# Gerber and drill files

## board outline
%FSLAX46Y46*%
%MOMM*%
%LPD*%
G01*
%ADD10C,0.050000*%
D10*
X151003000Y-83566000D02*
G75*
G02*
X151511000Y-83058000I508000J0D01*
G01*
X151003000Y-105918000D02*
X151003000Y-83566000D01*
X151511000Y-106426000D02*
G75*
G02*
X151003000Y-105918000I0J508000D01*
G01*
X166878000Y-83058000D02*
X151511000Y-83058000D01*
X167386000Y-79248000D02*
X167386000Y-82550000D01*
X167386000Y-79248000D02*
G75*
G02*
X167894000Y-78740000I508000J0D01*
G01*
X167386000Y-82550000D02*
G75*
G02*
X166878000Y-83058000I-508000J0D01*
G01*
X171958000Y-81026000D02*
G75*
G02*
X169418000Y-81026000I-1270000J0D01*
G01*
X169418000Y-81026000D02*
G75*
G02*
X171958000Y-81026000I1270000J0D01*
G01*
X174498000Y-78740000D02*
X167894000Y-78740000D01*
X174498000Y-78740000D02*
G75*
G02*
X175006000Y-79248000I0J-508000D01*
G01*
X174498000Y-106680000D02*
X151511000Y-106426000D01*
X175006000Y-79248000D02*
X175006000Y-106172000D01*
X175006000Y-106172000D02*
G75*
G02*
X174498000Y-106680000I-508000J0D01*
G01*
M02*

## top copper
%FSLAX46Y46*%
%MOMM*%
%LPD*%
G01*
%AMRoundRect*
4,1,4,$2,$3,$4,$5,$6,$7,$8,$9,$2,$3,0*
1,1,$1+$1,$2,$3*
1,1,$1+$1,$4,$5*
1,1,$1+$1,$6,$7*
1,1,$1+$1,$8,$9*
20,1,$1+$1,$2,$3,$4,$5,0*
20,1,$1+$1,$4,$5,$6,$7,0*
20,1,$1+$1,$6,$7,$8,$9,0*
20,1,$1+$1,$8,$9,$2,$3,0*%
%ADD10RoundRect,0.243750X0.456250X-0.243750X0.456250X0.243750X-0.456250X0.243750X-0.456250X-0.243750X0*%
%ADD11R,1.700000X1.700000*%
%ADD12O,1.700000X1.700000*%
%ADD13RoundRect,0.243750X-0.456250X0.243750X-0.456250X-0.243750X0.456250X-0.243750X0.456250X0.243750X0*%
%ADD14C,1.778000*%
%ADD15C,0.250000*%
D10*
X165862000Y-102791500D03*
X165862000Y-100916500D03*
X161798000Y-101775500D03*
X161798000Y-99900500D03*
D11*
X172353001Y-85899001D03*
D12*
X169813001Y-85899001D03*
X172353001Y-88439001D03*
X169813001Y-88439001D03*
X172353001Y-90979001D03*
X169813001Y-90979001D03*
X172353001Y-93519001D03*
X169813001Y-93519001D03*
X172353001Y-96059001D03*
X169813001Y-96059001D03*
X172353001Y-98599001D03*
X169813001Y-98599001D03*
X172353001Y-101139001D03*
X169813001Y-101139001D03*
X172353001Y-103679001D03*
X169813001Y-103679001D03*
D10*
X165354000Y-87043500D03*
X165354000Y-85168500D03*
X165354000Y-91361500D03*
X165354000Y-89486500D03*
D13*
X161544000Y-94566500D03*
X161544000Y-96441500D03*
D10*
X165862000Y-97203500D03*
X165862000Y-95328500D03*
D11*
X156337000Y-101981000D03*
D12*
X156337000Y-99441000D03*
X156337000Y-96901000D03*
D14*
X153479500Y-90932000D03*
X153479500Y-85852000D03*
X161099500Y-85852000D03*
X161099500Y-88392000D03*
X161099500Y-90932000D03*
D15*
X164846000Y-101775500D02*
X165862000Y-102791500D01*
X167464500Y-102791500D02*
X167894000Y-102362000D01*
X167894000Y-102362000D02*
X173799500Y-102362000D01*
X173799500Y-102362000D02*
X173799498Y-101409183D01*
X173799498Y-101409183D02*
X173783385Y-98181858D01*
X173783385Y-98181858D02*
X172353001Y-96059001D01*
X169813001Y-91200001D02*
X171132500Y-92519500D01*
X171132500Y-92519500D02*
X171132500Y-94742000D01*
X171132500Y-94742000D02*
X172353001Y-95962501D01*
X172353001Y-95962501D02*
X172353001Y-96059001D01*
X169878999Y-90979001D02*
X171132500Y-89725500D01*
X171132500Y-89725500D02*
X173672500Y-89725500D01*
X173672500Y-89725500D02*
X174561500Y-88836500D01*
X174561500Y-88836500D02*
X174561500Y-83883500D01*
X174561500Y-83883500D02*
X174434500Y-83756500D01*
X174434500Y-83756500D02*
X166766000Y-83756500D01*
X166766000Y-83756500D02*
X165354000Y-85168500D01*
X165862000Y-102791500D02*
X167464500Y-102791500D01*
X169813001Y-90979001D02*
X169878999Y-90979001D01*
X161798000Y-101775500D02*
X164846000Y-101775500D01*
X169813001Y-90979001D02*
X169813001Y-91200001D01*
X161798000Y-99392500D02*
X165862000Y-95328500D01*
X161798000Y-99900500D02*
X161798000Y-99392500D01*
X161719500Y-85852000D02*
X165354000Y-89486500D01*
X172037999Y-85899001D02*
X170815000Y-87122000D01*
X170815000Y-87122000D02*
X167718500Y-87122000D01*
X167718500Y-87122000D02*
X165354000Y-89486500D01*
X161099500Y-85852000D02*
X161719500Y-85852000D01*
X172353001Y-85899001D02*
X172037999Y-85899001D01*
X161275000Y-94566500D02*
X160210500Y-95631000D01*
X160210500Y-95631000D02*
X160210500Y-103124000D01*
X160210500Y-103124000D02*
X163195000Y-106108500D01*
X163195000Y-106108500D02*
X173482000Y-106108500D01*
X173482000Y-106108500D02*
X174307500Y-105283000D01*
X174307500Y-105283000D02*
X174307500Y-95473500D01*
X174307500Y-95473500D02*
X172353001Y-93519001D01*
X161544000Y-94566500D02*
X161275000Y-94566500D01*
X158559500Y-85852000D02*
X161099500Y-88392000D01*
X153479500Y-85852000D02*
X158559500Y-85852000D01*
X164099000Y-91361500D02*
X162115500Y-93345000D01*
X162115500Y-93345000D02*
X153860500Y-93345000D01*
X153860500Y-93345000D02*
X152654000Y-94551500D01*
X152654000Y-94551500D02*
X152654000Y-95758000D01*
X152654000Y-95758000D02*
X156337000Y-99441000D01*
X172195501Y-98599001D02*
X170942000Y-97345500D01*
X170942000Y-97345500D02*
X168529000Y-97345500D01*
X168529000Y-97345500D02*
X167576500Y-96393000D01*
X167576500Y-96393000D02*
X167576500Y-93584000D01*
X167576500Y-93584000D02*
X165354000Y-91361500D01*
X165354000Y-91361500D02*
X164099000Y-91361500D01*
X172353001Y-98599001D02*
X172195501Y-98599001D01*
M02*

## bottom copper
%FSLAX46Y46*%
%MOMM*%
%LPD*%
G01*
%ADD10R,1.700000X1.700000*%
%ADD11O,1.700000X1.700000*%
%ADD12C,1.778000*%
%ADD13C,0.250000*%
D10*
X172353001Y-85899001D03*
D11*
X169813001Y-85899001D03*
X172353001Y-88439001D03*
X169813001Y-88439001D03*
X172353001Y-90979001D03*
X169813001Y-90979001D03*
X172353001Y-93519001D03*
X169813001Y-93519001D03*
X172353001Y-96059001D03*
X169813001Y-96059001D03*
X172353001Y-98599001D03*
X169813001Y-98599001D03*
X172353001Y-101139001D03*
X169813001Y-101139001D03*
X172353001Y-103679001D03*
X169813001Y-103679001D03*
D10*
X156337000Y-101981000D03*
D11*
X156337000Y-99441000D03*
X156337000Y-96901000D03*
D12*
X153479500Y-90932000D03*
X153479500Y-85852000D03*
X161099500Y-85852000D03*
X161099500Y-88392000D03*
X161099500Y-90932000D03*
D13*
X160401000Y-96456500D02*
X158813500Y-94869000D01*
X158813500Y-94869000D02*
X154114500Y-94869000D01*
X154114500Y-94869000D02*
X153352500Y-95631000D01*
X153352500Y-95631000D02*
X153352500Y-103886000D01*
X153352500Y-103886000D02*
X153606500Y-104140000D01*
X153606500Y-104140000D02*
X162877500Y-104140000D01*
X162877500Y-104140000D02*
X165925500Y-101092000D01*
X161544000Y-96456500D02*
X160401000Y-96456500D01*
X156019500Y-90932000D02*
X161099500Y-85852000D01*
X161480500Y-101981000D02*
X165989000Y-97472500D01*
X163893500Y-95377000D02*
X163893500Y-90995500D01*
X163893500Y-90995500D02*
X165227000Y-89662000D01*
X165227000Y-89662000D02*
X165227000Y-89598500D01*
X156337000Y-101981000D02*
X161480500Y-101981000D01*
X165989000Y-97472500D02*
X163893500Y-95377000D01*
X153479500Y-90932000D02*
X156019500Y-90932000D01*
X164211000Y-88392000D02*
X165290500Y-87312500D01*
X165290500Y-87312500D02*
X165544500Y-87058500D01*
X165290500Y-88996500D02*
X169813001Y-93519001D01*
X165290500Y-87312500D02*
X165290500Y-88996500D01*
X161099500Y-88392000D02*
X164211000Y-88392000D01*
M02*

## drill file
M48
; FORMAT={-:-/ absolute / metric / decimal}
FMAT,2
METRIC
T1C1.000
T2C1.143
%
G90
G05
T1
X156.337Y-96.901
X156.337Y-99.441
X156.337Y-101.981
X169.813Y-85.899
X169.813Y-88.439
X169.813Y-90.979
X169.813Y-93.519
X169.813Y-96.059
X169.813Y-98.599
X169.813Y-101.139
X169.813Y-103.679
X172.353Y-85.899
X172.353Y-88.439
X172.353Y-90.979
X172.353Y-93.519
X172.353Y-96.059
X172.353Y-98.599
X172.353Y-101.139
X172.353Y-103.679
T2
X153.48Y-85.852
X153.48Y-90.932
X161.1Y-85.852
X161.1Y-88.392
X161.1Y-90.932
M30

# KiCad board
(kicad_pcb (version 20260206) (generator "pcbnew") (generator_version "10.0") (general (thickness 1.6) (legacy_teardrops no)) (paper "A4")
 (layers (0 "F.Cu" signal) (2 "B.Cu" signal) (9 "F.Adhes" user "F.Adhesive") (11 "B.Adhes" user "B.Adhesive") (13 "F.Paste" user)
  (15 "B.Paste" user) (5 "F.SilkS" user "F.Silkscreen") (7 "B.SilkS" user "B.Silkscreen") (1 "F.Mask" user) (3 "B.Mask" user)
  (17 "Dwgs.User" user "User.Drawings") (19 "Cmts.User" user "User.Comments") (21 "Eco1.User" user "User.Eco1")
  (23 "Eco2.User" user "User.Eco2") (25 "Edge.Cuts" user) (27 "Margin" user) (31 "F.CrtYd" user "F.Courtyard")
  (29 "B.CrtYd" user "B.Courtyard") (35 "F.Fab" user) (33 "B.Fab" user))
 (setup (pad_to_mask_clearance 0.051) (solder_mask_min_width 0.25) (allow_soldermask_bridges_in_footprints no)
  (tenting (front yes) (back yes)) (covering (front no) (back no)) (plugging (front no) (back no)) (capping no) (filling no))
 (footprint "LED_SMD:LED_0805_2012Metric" (layer "F.Cu") (at 165.862 101.854 90)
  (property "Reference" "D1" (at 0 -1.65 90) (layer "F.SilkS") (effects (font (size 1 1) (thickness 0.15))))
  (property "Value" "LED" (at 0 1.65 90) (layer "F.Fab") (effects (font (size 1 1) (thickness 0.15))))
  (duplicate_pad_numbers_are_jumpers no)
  (pad "1" smd roundrect (at -0.9375 0 90) (size 0.975 1.4) (layers "F.Cu" "F.Mask" "F.Paste") (roundrect_rratio 0.25) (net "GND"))
  (pad "2" smd roundrect (at 0.9375 0 90) (size 0.975 1.4) (layers "F.Cu" "F.Mask" "F.Paste") (roundrect_rratio 0.25) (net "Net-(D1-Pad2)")))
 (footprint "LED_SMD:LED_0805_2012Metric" (layer "F.Cu") (at 161.798 100.838 90)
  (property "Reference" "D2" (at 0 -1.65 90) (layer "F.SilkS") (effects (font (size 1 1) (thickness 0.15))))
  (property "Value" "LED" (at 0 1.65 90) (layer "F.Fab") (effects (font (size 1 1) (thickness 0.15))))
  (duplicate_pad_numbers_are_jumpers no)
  (pad "1" smd roundrect (at -0.9375 0 90) (size 0.975 1.4) (layers "F.Cu" "F.Mask" "F.Paste") (roundrect_rratio 0.25) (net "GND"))
  (pad "2" smd roundrect (at 0.9375 0 90) (size 0.975 1.4) (layers "F.Cu" "F.Mask" "F.Paste") (roundrect_rratio 0.25) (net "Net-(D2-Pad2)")))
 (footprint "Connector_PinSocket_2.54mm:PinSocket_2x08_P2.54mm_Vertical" (layer "F.Cu") (at 172.353001 85.899001)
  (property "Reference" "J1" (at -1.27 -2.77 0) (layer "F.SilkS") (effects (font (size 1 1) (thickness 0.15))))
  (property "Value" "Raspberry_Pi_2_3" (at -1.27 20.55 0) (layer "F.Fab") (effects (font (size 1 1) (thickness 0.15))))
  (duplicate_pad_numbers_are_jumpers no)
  (pad "1" thru_hole rect (at 0 0) (size 1.7 1.7) (drill 1) (layers "*.Cu" "*.Mask") (remove_unused_layers no) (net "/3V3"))
  (pad "2" thru_hole oval (at -2.54 0) (size 1.7 1.7) (drill 1) (layers "*.Cu" "*.Mask") (remove_unused_layers no) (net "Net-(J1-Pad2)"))
  (pad "3" thru_hole oval (at 0 2.54) (size 1.7 1.7) (drill 1) (layers "*.Cu" "*.Mask") (remove_unused_layers no) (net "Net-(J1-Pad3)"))
  (pad "4" thru_hole oval (at -2.54 2.54) (size 1.7 1.7) (drill 1) (layers "*.Cu" "*.Mask") (remove_unused_layers no) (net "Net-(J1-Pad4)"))
  (pad "5" thru_hole oval (at 0 5.08) (size 1.7 1.7) (drill 1) (layers "*.Cu" "*.Mask") (remove_unused_layers no) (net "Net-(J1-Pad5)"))
  (pad "6" thru_hole oval (at -2.54 5.08) (size 1.7 1.7) (drill 1) (layers "*.Cu" "*.Mask") (remove_unused_layers no) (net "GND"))
  (pad "7" thru_hole oval (at 0 7.62) (size 1.7 1.7) (drill 1) (layers "*.Cu" "*.Mask") (remove_unused_layers no) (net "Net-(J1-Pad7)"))
  (pad "8" thru_hole oval (at -2.54 7.62) (size 1.7 1.7) (drill 1) (layers "*.Cu" "*.Mask") (remove_unused_layers no) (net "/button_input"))
  (pad "9" thru_hole oval (at 0 10.16) (size 1.7 1.7) (drill 1) (layers "*.Cu" "*.Mask") (remove_unused_layers no) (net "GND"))
  (pad "10" thru_hole oval (at -2.54 10.16) (size 1.7 1.7) (drill 1) (layers "*.Cu" "*.Mask") (remove_unused_layers no)
   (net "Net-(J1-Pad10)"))
  (pad "11" thru_hole oval (at 0 12.7) (size 1.7 1.7) (drill 1) (layers "*.Cu" "*.Mask") (remove_unused_layers no) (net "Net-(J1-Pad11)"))
  (pad "12" thru_hole oval (at -2.54 12.7) (size 1.7 1.7) (drill 1) (layers "*.Cu" "*.Mask") (remove_unused_layers no)
   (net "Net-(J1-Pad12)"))
  (pad "13" thru_hole oval (at 0 15.24) (size 1.7 1.7) (drill 1) (layers "*.Cu" "*.Mask") (remove_unused_layers no) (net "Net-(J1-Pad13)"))
  (pad "14" thru_hole oval (at -2.54 15.24) (size 1.7 1.7) (drill 1) (layers "*.Cu" "*.Mask") (remove_unused_layers no)
   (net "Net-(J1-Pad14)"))
  (pad "15" thru_hole oval (at 0 17.78) (size 1.7 1.7) (drill 1) (layers "*.Cu" "*.Mask") (remove_unused_layers no) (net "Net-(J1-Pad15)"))
  (pad "16" thru_hole oval (at -2.54 17.78) (size 1.7 1.7) (drill 1) (layers "*.Cu" "*.Mask") (remove_unused_layers no)
   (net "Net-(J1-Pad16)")))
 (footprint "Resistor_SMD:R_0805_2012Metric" (layer "F.Cu") (at 165.354 86.106 90)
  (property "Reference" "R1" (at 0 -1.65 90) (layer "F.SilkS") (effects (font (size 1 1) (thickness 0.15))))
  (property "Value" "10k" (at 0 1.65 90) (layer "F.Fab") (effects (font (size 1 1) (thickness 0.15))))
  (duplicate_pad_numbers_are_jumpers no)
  (pad "1" smd roundrect (at -0.9375 0 90) (size 0.975 1.4) (layers "F.Cu" "F.Mask" "F.Paste") (roundrect_rratio 0.25) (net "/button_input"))
  (pad "2" smd roundrect (at 0.9375 0 90) (size 0.975 1.4) (layers "F.Cu" "F.Mask" "F.Paste") (roundrect_rratio 0.25) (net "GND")))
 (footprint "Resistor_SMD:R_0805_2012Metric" (layer "F.Cu") (at 165.354 90.424 90)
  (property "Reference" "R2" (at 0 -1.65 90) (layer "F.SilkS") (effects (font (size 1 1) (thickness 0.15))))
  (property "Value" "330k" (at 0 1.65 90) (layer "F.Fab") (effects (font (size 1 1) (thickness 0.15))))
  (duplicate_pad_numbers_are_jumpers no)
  (pad "1" smd roundrect (at -0.9375 0 90) (size 0.975 1.4) (layers "F.Cu" "F.Mask" "F.Paste") (roundrect_rratio 0.25)
   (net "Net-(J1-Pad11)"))
  (pad "2" smd roundrect (at 0.9375 0 90) (size 0.975 1.4) (layers "F.Cu" "F.Mask" "F.Paste") (roundrect_rratio 0.25) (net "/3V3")))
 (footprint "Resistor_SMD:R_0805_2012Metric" (layer "F.Cu") (at 161.544 95.504 -90)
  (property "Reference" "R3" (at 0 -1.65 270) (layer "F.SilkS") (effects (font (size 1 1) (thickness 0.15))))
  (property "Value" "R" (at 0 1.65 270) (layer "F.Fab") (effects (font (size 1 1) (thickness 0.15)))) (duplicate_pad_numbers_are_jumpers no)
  (pad "1" smd roundrect (at -0.9375 0 270) (size 0.975 1.4) (layers "F.Cu" "F.Mask" "F.Paste") (roundrect_rratio 0.25)
   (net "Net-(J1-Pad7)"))
  (pad "2" smd roundrect (at 0.9375 0 270) (size 0.975 1.4) (layers "F.Cu" "F.Mask" "F.Paste") (roundrect_rratio 0.25) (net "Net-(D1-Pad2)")))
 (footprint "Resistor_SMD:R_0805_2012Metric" (layer "F.Cu") (at 165.862 96.266 90)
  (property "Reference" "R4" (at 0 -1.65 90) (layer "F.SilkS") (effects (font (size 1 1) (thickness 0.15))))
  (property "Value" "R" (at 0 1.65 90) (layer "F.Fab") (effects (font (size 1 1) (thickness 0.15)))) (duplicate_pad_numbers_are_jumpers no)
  (pad "1" smd roundrect (at -0.9375 0 90) (size 0.975 1.4) (layers "F.Cu" "F.Mask" "F.Paste") (roundrect_rratio 0.25) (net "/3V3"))
  (pad "2" smd roundrect (at 0.9375 0 90) (size 0.975 1.4) (layers "F.Cu" "F.Mask" "F.Paste") (roundrect_rratio 0.25) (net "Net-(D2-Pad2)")))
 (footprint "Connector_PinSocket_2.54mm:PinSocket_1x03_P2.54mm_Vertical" (layer "F.Cu") (at 156.337 101.981 180)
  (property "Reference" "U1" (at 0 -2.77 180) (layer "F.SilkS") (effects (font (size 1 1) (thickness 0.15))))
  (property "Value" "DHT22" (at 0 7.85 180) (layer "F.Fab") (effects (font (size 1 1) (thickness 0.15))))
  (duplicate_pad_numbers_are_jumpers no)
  (pad "1" thru_hole rect (at 0 0 180) (size 1.7 1.7) (drill 1) (layers "*.Cu" "*.Mask") (remove_unused_layers no) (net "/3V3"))
  (pad "2" thru_hole oval (at 0 2.54 180) (size 1.7 1.7) (drill 1) (layers "*.Cu" "*.Mask") (remove_unused_layers no) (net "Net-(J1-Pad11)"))
  (pad "3" thru_hole oval (at 0 5.08 180) (size 1.7 1.7) (drill 1) (layers "*.Cu" "*.Mask") (remove_unused_layers no) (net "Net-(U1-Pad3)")))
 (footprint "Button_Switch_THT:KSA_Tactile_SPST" (layer "F.Cu") (at 153.4795 90.932 90)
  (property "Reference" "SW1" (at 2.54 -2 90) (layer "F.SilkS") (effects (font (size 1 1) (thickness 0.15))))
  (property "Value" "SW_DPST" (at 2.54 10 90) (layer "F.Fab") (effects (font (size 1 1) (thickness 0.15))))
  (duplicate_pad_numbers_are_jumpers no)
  (pad "1" thru_hole circle (at 0 0 90) (size 1.778 1.778) (drill 1.143) (layers "*.Cu" "*.Mask") (remove_unused_layers no) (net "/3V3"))
  (pad "2" thru_hole circle (at 5.08 0 90) (size 1.778 1.778) (drill 1.143) (layers "*.Cu" "*.Mask") (remove_unused_layers no)
   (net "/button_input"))
  (pad "3" thru_hole circle (at 5.08 7.62 90) (size 1.778 1.778) (drill 1.143) (layers "*.Cu" "*.Mask") (remove_unused_layers no)
   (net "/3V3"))
  (pad "4" thru_hole circle (at 2.54 7.62 90) (size 1.778 1.778) (drill 1.143) (layers "*.Cu" "*.Mask") (remove_unused_layers no)
   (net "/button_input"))
  (pad "5" thru_hole circle (at 0 7.62 90) (size 1.778 1.778) (drill 1.143) (layers "*.Cu" "*.Mask") (remove_unused_layers no)))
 (gr_arc (start 151.003 83.566) (mid 151.15179 83.20679) (end 151.511 83.058) (stroke (width 0.05) (type solid)) (layer "Edge.Cuts"))
 (gr_line (start 151.003 105.918) (end 151.003 83.566) (stroke (width 0.05) (type solid)) (layer "Edge.Cuts"))
 (gr_arc (start 151.511 106.426) (mid 151.15179 106.27721) (end 151.003 105.918) (stroke (width 0.05) (type solid)) (layer "Edge.Cuts"))
 (gr_line (start 166.878 83.058) (end 151.511 83.058) (stroke (width 0.05) (type solid)) (layer "Edge.Cuts"))
 (gr_line (start 167.386 79.248) (end 167.386 82.55) (stroke (width 0.05) (type solid)) (layer "Edge.Cuts"))
 (gr_arc (start 167.386 79.248) (mid 167.53479 78.88879) (end 167.894 78.74) (stroke (width 0.05) (type solid)) (layer "Edge.Cuts"))
 (gr_arc (start 167.386 82.55) (mid 167.23721 82.90921) (end 166.878 83.058) (stroke (width 0.05) (type solid)) (layer "Edge.Cuts"))
 (gr_circle (center 170.688 81.026) (end 171.704 81.788) (stroke (width 0.05) (type solid)) (fill no) (layer "Edge.Cuts"))
 (gr_line (start 174.498 78.74) (end 167.894 78.74) (stroke (width 0.05) (type solid)) (layer "Edge.Cuts"))
 (gr_arc (start 174.498 78.74) (mid 174.85721 78.88879) (end 175.006 79.248) (stroke (width 0.05) (type solid)) (layer "Edge.Cuts"))
 (gr_line (start 174.498 106.68) (end 151.511 106.426) (stroke (width 0.05) (type solid)) (layer "Edge.Cuts"))
 (gr_line (start 175.006 79.248) (end 175.006 106.172) (stroke (width 0.05) (type solid)) (layer "Edge.Cuts"))
 (gr_arc (start 175.006 106.172) (mid 174.85721 106.53121) (end 174.498 106.68) (stroke (width 0.05) (type solid)) (layer "Edge.Cuts"))
 (segment (start 160.401 96.4565) (end 158.8135 94.869) (width 0.25) (layer "B.Cu") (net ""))
 (segment (start 158.8135 94.869) (end 154.1145 94.869) (width 0.25) (layer "B.Cu") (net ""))
 (segment (start 154.1145 94.869) (end 153.3525 95.631) (width 0.25) (layer "B.Cu") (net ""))
 (segment (start 153.3525 95.631) (end 153.3525 103.886) (width 0.25) (layer "B.Cu") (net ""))
 (segment (start 153.3525 103.886) (end 153.6065 104.14) (width 0.25) (layer "B.Cu") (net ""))
 (segment (start 153.6065 104.14) (end 162.8775 104.14) (width 0.25) (layer "B.Cu") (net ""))
 (segment (start 162.8775 104.14) (end 165.9255 101.092) (width 0.25) (layer "B.Cu") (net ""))
 (segment (start 161.544 96.4565) (end 160.401 96.4565) (width 0.25) (layer "B.Cu") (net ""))
 (segment (start 164.846 101.7755) (end 165.862 102.7915) (width 0.25) (layer "F.Cu") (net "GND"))
 (segment (start 167.4645 102.7915) (end 167.894 102.362) (width 0.25) (layer "F.Cu") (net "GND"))
 (segment (start 167.894 102.362) (end 173.7995 102.362) (width 0.25) (layer "F.Cu") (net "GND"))
 (segment (start 173.7995 102.362) (end 173.799498 101.409183) (width 0.25) (layer "F.Cu") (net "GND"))
 (segment (start 173.799498 101.409183) (end 173.783385 98.181858) (width 0.25) (layer "F.Cu") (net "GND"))
 (segment (start 173.783385 98.181858) (end 172.353001 96.059001) (width 0.25) (layer "F.Cu") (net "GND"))
 (segment (start 169.813001 91.200001) (end 171.1325 92.5195) (width 0.25) (layer "F.Cu") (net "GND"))
 (segment (start 171.1325 92.5195) (end 171.1325 94.742) (width 0.25) (layer "F.Cu") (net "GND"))
 (segment (start 171.1325 94.742) (end 172.353001 95.962501) (width 0.25) (layer "F.Cu") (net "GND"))
 (segment (start 172.353001 95.962501) (end 172.353001 96.059001) (width 0.25) (layer "F.Cu") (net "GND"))
 (segment (start 169.878999 90.979001) (end 171.1325 89.7255) (width 0.25) (layer "F.Cu") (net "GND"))
 (segment (start 171.1325 89.7255) (end 173.6725 89.7255) (width 0.25) (layer "F.Cu") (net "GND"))
 (segment (start 173.6725 89.7255) (end 174.5615 88.8365) (width 0.25) (layer "F.Cu") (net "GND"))
 (segment (start 174.5615 88.8365) (end 174.5615 83.8835) (width 0.25) (layer "F.Cu") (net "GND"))
 (segment (start 174.5615 83.8835) (end 174.4345 83.7565) (width 0.25) (layer "F.Cu") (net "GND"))
 (segment (start 174.4345 83.7565) (end 166.766 83.7565) (width 0.25) (layer "F.Cu") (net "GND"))
 (segment (start 166.766 83.7565) (end 165.354 85.1685) (width 0.25) (layer "F.Cu") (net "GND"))
 (segment (start 165.862 102.7915) (end 167.4645 102.7915) (width 0.25) (layer "F.Cu") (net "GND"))
 (segment (start 169.813001 90.979001) (end 169.878999 90.979001) (width 0.25) (layer "F.Cu") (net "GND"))
 (segment (start 161.798 101.7755) (end 164.846 101.7755) (width 0.25) (layer "F.Cu") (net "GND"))
 (segment (start 169.813001 90.979001) (end 169.813001 91.200001) (width 0.25) (layer "F.Cu") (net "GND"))
 (segment (start 161.798 99.3925) (end 165.862 95.3285) (width 0.25) (layer "F.Cu") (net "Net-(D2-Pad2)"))
 (segment (start 161.798 99.9005) (end 161.798 99.3925) (width 0.25) (layer "F.Cu") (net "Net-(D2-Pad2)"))
 (segment (start 161.7195 85.852) (end 165.354 89.4865) (width 0.25) (layer "F.Cu") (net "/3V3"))
 (segment (start 172.037999 85.899001) (end 170.815 87.122) (width 0.25) (layer "F.Cu") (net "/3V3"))
 (segment (start 170.815 87.122) (end 167.7185 87.122) (width 0.25) (layer "F.Cu") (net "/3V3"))
 (segment (start 167.7185 87.122) (end 165.354 89.4865) (width 0.25) (layer "F.Cu") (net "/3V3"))
 (segment (start 161.0995 85.852) (end 161.7195 85.852) (width 0.25) (layer "F.Cu") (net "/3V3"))
 (segment (start 172.353001 85.899001) (end 172.037999 85.899001) (width 0.25) (layer "F.Cu") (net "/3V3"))
 (segment (start 156.0195 90.932) (end 161.0995 85.852) (width 0.25) (layer "B.Cu") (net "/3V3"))
 (segment (start 161.4805 101.981) (end 165.989 97.4725) (width 0.25) (layer "B.Cu") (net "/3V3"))
 (segment (start 163.8935 95.377) (end 163.8935 90.9955) (width 0.25) (layer "B.Cu") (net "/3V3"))
 (segment (start 163.8935 90.9955) (end 165.227 89.662) (width 0.25) (layer "B.Cu") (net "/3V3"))
 (segment (start 165.227 89.662) (end 165.227 89.5985) (width 0.25) (layer "B.Cu") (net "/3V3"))
 (segment (start 156.337 101.981) (end 161.4805 101.981) (width 0.25) (layer "B.Cu") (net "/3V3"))
 (segment (start 165.989 97.4725) (end 163.8935 95.377) (width 0.25) (layer "B.Cu") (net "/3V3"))
 (segment (start 153.4795 90.932) (end 156.0195 90.932) (width 0.25) (layer "B.Cu") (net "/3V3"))
 (segment (start 161.275 94.5665) (end 160.2105 95.631) (width 0.25) (layer "F.Cu") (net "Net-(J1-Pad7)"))
 (segment (start 160.2105 95.631) (end 160.2105 103.124) (width 0.25) (layer "F.Cu") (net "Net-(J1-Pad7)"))
 (segment (start 160.2105 103.124) (end 163.195 106.1085) (width 0.25) (layer "F.Cu") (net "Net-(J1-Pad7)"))
 (segment (start 163.195 106.1085) (end 173.482 106.1085) (width 0.25) (layer "F.Cu") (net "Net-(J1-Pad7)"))
 (segment (start 173.482 106.1085) (end 174.3075 105.283) (width 0.25) (layer "F.Cu") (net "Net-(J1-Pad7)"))
 (segment (start 174.3075 105.283) (end 174.3075 95.4735) (width 0.25) (layer "F.Cu") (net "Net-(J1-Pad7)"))
 (segment (start 174.3075 95.4735) (end 172.353001 93.519001) (width 0.25) (layer "F.Cu") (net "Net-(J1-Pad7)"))
 (segment (start 161.544 94.5665) (end 161.275 94.5665) (width 0.25) (layer "F.Cu") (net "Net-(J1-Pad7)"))
 (segment (start 158.5595 85.852) (end 161.0995 88.392) (width 0.25) (layer "F.Cu") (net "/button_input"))
 (segment (start 153.4795 85.852) (end 158.5595 85.852) (width 0.25) (layer "F.Cu") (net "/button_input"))
 (segment (start 164.211 88.392) (end 165.2905 87.3125) (width 0.25) (layer "B.Cu") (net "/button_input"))
 (segment (start 165.2905 87.3125) (end 165.5445 87.0585) (width 0.25) (layer "B.Cu") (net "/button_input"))
 (segment (start 165.2905 88.9965) (end 169.813001 93.519001) (width 0.25) (layer "B.Cu") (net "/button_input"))
 (segment (start 165.2905 87.3125) (end 165.2905 88.9965) (width 0.25) (layer "B.Cu") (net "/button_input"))
 (segment (start 161.0995 88.392) (end 164.211 88.392) (width 0.25) (layer "B.Cu") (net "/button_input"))
 (segment (start 164.099 91.3615) (end 162.1155 93.345) (width 0.25) (layer "F.Cu") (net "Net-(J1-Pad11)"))
 (segment (start 162.1155 93.345) (end 153.8605 93.345) (width 0.25) (layer "F.Cu") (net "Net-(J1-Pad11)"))
 (segment (start 153.8605 93.345) (end 152.654 94.5515) (width 0.25) (layer "F.Cu") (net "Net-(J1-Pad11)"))
 (segment (start 152.654 94.5515) (end 152.654 95.758) (width 0.25) (layer "F.Cu") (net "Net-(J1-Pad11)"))
 (segment (start 152.654 95.758) (end 156.337 99.441) (width 0.25) (layer "F.Cu") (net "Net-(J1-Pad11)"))
 (segment (start 172.195501 98.599001) (end 170.942 97.3455) (width 0.25) (layer "F.Cu") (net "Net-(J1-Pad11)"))
 (segment (start 170.942 97.3455) (end 168.529 97.3455) (width 0.25) (layer "F.Cu") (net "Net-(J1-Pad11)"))
 (segment (start 168.529 97.3455) (end 167.5765 96.393) (width 0.25) (layer "F.Cu") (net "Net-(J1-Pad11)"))
 (segment (start 167.5765 96.393) (end 167.5765 93.584) (width 0.25) (layer "F.Cu") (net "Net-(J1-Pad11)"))
 (segment (start 167.5765 93.584) (end 165.354 91.3615) (width 0.25) (layer "F.Cu") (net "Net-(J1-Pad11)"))
 (segment (start 165.354 91.3615) (end 164.099 91.3615) (width 0.25) (layer "F.Cu") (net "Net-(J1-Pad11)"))
 (segment (start 172.353001 98.599001) (end 172.195501 98.599001) (width 0.25) (layer "F.Cu") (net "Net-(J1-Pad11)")))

